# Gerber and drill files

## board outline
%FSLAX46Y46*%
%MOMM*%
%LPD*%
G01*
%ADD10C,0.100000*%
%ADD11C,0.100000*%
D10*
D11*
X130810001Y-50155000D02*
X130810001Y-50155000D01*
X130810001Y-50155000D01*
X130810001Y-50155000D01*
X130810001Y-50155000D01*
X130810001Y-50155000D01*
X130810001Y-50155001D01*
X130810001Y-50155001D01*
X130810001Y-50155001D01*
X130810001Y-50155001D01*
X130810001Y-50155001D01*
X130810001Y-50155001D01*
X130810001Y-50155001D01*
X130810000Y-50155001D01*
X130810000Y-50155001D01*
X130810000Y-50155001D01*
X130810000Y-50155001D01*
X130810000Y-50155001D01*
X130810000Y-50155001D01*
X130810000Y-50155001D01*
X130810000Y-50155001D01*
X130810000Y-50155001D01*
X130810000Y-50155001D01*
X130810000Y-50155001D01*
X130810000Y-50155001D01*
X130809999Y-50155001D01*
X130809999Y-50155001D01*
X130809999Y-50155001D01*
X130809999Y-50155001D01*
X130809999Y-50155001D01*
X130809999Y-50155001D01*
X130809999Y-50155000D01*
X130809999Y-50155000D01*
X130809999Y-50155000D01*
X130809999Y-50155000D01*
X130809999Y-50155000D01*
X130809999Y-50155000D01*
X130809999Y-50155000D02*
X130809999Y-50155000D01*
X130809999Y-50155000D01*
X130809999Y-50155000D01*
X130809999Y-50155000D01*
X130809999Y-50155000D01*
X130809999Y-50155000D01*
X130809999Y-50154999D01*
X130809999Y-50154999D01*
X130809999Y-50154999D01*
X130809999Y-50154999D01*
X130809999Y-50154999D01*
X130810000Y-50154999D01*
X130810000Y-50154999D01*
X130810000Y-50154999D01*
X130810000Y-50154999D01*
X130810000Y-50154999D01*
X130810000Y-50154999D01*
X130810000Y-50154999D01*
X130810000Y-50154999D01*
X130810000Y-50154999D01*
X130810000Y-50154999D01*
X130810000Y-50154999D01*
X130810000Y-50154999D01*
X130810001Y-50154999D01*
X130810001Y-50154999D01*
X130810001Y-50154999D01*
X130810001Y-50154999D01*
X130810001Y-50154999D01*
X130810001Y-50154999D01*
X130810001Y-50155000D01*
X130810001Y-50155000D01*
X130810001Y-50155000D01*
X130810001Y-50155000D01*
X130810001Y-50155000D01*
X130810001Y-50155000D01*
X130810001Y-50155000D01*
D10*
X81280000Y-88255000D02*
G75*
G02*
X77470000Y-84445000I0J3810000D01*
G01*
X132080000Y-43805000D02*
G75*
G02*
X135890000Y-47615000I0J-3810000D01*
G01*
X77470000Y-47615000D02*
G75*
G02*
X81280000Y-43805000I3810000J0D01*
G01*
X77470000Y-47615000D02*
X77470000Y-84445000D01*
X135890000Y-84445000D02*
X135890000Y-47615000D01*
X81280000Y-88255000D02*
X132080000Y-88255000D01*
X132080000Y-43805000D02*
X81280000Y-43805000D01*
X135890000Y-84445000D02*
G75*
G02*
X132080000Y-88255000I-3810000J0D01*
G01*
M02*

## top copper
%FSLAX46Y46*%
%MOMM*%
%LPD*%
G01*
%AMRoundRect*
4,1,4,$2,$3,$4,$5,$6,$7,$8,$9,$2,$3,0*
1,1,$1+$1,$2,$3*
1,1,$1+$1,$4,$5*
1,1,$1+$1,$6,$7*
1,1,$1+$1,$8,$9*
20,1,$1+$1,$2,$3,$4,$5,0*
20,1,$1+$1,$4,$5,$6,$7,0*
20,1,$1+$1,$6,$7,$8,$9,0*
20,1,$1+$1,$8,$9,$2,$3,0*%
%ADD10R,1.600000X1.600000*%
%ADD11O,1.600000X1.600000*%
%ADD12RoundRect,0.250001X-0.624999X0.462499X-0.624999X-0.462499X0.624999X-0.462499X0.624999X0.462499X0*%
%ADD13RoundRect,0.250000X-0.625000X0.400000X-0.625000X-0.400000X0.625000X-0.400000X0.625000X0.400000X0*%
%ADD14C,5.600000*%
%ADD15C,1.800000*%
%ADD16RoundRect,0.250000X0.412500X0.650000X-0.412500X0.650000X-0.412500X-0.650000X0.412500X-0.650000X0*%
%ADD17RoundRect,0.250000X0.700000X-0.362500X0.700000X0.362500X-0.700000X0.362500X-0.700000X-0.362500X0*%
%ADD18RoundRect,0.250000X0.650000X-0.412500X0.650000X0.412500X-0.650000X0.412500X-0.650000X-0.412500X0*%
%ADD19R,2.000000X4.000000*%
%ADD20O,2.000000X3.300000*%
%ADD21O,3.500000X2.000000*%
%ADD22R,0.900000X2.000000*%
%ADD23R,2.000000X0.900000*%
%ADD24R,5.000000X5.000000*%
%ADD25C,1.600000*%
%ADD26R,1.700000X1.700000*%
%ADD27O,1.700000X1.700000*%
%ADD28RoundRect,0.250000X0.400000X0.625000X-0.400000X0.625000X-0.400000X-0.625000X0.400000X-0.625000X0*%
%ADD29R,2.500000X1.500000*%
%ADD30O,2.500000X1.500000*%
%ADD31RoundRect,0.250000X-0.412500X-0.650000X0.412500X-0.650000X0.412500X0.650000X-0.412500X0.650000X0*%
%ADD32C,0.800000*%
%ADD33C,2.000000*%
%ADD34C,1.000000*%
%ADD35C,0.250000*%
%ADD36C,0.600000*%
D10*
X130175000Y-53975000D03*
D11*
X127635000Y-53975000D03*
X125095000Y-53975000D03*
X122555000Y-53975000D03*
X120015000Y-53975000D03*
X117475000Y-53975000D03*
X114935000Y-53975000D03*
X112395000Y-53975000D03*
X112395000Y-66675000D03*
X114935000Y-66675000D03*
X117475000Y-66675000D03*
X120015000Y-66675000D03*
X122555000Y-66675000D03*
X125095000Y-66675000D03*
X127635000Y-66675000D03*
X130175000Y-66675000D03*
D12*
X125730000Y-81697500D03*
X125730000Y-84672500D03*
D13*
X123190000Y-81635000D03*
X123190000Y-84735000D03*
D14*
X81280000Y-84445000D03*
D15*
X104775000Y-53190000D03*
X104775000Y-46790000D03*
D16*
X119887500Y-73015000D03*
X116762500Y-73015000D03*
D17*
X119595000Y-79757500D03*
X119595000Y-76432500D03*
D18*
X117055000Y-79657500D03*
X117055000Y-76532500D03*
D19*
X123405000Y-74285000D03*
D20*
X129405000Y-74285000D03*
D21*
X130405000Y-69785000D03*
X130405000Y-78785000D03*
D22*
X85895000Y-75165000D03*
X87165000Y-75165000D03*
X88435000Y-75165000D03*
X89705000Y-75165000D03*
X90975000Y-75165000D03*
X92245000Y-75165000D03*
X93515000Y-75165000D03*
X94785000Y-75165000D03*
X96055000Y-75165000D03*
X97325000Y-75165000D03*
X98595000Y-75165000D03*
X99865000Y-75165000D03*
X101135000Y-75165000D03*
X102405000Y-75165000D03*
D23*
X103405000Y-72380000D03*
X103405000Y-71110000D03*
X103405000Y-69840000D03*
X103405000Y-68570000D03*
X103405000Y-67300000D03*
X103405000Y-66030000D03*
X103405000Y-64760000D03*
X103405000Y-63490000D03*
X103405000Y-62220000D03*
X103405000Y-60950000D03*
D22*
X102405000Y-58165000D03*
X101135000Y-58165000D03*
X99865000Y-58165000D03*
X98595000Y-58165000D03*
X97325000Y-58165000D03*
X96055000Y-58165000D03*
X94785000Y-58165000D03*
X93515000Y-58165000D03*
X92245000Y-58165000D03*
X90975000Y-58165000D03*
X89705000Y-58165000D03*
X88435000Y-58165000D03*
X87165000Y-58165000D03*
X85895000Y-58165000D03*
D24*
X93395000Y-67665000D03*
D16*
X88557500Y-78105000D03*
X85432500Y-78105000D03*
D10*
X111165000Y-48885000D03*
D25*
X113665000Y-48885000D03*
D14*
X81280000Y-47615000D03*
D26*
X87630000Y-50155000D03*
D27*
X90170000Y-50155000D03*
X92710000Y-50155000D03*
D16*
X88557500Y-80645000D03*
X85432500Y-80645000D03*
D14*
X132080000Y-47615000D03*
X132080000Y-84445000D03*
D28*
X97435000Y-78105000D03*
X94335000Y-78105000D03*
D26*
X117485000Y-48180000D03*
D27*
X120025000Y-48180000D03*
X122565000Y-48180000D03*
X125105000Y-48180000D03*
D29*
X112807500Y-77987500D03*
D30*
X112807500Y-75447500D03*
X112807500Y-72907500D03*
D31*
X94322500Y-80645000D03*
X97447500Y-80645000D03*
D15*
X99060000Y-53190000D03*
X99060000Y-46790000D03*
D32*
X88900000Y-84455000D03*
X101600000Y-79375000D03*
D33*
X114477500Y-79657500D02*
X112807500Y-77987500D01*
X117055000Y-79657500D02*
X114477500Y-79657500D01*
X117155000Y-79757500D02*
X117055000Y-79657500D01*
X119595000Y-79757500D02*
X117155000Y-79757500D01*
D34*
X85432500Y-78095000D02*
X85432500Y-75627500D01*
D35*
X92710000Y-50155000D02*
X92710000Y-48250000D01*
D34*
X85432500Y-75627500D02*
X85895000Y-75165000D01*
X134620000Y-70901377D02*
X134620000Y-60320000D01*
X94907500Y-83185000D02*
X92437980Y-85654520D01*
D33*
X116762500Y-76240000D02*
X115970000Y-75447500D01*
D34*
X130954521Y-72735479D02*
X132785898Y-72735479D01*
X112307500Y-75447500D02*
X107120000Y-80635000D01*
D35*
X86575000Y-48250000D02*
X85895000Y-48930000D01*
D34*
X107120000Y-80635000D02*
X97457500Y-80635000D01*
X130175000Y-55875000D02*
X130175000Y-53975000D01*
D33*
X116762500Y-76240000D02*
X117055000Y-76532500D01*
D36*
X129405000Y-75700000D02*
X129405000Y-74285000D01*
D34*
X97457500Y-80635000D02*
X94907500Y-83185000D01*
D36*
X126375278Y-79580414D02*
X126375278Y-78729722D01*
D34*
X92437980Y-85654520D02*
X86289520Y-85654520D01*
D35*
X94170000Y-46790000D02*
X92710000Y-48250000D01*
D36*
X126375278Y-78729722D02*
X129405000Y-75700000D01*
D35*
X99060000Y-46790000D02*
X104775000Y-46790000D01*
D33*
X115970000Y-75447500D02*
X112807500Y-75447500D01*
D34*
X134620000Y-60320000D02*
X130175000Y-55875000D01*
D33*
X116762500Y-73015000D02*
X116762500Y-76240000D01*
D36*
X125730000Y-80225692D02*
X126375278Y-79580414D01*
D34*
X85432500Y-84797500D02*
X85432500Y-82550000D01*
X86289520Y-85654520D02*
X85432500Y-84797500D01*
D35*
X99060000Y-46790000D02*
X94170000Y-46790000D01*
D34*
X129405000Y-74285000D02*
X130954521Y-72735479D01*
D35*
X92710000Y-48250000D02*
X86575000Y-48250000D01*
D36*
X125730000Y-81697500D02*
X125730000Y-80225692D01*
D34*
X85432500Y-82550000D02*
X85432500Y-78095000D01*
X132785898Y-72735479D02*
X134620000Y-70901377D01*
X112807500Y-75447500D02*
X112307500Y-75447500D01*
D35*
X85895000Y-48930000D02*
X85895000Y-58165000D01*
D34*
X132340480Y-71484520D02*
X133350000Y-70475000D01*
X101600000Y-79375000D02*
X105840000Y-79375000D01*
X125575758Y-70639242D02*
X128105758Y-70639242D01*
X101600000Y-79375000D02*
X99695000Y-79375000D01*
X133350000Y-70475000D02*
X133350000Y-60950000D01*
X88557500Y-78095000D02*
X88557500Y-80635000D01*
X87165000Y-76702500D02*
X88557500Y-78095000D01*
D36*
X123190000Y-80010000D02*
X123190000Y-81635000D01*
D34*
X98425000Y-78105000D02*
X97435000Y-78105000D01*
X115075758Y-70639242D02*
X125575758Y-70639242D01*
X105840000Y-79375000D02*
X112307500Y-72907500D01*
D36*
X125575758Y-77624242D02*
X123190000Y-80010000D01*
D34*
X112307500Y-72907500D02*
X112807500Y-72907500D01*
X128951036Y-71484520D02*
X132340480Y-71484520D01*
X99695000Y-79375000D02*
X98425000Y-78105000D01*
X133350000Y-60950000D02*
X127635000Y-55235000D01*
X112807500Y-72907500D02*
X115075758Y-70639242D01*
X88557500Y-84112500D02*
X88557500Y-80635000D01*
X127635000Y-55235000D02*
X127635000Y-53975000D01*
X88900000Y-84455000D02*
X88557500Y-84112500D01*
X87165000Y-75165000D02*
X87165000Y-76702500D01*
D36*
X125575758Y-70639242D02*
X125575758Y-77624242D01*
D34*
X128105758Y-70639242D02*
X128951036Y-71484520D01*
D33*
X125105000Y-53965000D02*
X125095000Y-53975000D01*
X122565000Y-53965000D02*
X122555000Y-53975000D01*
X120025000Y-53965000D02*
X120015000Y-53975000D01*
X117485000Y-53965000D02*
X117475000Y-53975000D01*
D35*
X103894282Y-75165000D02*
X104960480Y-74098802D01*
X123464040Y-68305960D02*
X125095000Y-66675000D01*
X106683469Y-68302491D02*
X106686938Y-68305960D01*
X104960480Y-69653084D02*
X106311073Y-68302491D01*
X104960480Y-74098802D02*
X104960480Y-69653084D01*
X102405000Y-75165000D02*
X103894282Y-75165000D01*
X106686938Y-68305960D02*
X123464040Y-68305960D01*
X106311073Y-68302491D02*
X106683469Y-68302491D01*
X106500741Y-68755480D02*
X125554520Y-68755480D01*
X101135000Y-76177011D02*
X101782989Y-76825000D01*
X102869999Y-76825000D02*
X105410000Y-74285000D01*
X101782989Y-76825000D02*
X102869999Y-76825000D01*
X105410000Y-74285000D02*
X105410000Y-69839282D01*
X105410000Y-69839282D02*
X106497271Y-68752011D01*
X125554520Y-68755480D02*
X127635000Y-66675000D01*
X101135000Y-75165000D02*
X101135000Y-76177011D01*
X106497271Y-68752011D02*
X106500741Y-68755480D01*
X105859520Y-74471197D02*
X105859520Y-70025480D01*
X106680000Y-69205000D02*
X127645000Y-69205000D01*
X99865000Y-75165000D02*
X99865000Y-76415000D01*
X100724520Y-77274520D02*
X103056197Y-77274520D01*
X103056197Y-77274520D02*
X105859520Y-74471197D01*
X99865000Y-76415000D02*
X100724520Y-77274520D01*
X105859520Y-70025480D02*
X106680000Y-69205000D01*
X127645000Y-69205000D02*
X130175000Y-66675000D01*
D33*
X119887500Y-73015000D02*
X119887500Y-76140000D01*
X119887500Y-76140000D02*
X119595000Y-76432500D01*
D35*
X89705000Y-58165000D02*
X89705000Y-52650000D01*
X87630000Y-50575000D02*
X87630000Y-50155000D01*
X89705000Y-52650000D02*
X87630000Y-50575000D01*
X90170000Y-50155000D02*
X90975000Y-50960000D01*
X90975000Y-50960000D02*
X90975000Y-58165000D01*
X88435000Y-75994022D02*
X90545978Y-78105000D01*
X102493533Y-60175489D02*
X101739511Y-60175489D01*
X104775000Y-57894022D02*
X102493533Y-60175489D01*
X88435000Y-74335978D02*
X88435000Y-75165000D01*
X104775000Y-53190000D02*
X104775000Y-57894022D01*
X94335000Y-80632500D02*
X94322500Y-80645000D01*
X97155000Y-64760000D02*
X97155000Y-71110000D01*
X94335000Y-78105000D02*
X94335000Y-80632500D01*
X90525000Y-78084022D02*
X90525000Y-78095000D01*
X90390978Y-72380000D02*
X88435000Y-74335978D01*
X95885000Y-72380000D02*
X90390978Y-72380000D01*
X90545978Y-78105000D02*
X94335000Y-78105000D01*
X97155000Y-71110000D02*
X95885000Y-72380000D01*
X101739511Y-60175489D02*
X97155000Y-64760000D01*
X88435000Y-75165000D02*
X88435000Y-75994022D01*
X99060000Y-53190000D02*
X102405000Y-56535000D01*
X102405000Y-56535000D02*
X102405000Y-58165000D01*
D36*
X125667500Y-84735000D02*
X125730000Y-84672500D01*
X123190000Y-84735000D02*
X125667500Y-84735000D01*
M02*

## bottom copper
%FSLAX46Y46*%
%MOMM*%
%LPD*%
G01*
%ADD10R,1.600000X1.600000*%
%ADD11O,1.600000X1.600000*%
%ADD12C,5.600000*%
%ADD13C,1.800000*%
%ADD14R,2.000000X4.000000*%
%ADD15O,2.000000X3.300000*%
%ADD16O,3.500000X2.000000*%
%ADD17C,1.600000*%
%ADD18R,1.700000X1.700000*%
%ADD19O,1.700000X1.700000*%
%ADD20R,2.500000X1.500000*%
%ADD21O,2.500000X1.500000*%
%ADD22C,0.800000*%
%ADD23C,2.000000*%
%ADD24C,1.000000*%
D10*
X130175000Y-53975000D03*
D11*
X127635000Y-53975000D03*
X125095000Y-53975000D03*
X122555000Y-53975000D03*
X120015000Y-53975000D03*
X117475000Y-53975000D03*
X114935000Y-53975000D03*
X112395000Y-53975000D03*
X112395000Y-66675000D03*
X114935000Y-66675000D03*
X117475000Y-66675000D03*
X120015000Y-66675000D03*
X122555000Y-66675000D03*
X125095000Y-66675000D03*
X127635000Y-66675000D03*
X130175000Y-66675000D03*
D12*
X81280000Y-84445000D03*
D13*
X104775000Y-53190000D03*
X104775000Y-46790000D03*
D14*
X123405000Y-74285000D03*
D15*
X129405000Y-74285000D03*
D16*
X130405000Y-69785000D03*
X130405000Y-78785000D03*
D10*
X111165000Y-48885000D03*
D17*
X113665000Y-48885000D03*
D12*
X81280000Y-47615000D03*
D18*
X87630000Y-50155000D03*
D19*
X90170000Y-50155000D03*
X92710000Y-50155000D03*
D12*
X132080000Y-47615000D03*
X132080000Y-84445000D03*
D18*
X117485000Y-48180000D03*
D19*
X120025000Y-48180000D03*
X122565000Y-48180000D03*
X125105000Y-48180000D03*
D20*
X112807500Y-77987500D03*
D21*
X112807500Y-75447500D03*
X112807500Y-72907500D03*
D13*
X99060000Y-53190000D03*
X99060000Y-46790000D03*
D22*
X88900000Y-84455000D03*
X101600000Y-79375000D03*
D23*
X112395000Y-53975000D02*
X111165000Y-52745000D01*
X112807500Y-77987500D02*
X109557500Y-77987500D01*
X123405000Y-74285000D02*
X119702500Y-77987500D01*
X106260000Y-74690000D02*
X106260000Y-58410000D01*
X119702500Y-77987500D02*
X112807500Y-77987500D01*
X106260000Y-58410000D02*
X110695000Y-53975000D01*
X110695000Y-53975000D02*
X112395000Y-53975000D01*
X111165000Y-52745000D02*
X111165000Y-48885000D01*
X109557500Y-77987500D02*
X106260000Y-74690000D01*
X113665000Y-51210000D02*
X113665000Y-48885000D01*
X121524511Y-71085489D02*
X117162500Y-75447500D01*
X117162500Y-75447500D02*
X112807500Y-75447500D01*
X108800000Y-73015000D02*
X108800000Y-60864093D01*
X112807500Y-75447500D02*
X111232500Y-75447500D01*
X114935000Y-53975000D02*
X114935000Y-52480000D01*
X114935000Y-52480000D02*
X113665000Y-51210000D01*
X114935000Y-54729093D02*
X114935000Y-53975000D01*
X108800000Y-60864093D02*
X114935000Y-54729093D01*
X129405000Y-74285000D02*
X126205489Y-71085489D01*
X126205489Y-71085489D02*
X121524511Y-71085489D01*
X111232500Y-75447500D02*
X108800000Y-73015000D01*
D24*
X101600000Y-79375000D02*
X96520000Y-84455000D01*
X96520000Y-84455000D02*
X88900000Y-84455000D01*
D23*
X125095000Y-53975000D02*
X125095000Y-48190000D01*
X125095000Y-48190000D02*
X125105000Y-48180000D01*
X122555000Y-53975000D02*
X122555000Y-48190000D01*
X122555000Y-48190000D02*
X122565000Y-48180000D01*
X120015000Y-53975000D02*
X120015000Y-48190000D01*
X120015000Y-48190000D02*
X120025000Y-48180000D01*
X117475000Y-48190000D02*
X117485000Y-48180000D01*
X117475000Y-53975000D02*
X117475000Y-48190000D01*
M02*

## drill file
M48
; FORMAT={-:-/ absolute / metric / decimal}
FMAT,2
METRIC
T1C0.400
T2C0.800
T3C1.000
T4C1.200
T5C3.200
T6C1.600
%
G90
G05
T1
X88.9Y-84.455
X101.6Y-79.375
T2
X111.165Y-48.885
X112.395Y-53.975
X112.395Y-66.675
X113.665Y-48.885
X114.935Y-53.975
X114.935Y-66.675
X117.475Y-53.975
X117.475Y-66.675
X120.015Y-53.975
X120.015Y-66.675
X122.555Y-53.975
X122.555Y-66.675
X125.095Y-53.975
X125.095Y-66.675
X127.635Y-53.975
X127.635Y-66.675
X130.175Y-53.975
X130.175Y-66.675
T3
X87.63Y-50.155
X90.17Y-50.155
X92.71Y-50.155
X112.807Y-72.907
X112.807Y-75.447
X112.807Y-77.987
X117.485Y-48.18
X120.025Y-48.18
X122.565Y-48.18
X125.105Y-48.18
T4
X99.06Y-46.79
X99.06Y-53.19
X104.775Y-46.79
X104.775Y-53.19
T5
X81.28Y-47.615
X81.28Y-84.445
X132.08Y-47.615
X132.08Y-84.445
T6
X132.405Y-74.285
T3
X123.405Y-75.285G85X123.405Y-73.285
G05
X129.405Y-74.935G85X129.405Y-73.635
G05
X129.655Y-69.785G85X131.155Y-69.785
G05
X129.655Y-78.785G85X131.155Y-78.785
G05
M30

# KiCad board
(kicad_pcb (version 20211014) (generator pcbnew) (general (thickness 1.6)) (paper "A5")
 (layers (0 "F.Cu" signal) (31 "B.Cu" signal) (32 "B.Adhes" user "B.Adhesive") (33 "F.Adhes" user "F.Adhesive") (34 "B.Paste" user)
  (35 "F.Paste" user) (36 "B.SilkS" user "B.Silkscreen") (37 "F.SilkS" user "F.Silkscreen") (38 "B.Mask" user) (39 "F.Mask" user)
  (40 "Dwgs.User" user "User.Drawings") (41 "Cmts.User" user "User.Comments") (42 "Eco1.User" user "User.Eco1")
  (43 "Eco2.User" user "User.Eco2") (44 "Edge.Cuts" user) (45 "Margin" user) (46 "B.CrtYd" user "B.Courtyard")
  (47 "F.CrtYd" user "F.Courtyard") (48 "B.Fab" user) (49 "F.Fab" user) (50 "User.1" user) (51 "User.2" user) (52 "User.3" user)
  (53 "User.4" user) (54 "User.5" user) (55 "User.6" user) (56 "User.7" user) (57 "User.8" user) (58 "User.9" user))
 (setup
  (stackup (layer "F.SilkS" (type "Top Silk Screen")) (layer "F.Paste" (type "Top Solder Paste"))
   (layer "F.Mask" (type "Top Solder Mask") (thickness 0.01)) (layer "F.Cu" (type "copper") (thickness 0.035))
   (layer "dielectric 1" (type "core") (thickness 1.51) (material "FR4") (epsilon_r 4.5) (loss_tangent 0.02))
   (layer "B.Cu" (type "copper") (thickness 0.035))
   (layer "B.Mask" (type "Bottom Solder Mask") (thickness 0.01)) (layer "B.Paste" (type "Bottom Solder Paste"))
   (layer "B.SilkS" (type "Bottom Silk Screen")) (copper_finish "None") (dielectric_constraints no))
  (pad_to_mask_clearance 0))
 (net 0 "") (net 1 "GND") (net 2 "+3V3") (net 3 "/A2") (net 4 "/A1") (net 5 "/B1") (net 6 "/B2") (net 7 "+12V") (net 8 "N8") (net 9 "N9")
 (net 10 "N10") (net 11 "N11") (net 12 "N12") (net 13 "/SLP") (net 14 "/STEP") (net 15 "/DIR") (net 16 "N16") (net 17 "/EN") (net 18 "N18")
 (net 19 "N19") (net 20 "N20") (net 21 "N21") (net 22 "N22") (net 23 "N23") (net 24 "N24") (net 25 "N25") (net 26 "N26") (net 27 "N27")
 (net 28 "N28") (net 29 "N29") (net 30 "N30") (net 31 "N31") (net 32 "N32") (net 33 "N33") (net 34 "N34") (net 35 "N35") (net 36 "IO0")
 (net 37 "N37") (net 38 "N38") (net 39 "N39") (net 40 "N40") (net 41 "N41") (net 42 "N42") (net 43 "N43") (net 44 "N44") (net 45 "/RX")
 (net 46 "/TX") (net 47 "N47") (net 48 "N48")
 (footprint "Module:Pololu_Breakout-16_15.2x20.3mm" (layer "F.Cu") (at 130.175 53.975 -90)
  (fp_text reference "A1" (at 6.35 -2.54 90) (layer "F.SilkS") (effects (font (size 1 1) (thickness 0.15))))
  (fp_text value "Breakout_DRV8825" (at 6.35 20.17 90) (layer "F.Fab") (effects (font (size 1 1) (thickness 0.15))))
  (pad "1" thru_hole rect (at 0 0 270) (size 1.6 1.6) (drill 0.8) (layers *.Cu *.Mask) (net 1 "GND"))
  (pad "2" thru_hole oval (at 0 2.54 270) (size 1.6 1.6) (drill 0.8) (layers *.Cu *.Mask) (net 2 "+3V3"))
  (pad "3" thru_hole oval (at 0 5.08 270) (size 1.6 1.6) (drill 0.8) (layers *.Cu *.Mask) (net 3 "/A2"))
  (pad "4" thru_hole oval (at 0 7.62 270) (size 1.6 1.6) (drill 0.8) (layers *.Cu *.Mask) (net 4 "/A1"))
  (pad "5" thru_hole oval (at 0 10.16 270) (size 1.6 1.6) (drill 0.8) (layers *.Cu *.Mask) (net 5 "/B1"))
  (pad "6" thru_hole oval (at 0 12.7 270) (size 1.6 1.6) (drill 0.8) (layers *.Cu *.Mask) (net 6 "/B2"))
  (pad "7" thru_hole oval (at 0 15.24 270) (size 1.6 1.6) (drill 0.8) (layers *.Cu *.Mask) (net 1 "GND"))
  (pad "8" thru_hole oval (at 0 17.78 270) (size 1.6 1.6) (drill 0.8) (layers *.Cu *.Mask) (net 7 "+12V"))
  (pad "9" thru_hole oval (at 12.7 17.78 270) (size 1.6 1.6) (drill 0.8) (layers *.Cu *.Mask) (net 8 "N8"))
  (pad "10" thru_hole oval (at 12.7 15.24 270) (size 1.6 1.6) (drill 0.8) (layers *.Cu *.Mask) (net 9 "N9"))
  (pad "11" thru_hole oval (at 12.7 12.7 270) (size 1.6 1.6) (drill 0.8) (layers *.Cu *.Mask) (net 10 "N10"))
  (pad "12" thru_hole oval (at 12.7 10.16 270) (size 1.6 1.6) (drill 0.8) (layers *.Cu *.Mask) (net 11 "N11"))
  (pad "13" thru_hole oval (at 12.7 7.62 270) (size 1.6 1.6) (drill 0.8) (layers *.Cu *.Mask) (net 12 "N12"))
  (pad "14" thru_hole oval (at 12.7 5.08 270) (size 1.6 1.6) (drill 0.8) (layers *.Cu *.Mask) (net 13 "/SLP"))
  (pad "15" thru_hole oval (at 12.7 2.54 270) (size 1.6 1.6) (drill 0.8) (layers *.Cu *.Mask) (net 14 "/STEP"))
  (pad "16" thru_hole oval (at 12.7 0 270) (size 1.6 1.6) (drill 0.8) (layers *.Cu *.Mask) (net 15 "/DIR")))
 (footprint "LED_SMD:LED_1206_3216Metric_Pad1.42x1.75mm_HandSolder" (layer "F.Cu") (at 125.73 83.185 -90)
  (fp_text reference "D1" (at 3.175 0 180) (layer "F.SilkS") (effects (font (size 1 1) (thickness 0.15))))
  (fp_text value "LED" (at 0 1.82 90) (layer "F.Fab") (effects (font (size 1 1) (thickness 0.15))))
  (pad "1" smd roundrect (at -1.4875 0 270) (size 1.425 1.75) (layers "F.Cu" "F.Paste" "F.Mask") (roundrect_rratio 0.175439) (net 1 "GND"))
  (pad "2" smd roundrect (at 1.4875 0 270) (size 1.425 1.75) (layers "F.Cu" "F.Paste" "F.Mask") (roundrect_rratio 0.175439) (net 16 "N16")))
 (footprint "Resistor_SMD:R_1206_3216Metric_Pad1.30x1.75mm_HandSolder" (layer "F.Cu") (at 123.19 83.185 -90)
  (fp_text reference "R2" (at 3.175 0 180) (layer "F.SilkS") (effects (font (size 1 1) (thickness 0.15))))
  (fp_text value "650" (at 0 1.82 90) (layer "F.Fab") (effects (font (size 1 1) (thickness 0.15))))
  (pad "1" smd roundrect (at -1.55 0 270) (size 1.3 1.75) (layers "F.Cu" "F.Paste" "F.Mask") (roundrect_rratio 0.192308) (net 2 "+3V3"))
  (pad "2" smd roundrect (at 1.55 0 270) (size 1.3 1.75) (layers "F.Cu" "F.Paste" "F.Mask") (roundrect_rratio 0.192308) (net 16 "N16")))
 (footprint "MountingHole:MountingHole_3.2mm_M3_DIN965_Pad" (layer "F.Cu") (at 81.28 84.445)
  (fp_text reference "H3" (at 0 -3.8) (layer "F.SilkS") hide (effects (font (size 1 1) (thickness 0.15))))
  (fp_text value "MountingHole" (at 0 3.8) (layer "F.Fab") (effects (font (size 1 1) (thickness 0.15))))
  (pad "1" thru_hole circle (at 0 0) (size 5.6 5.6) (drill 3.2) (layers *.Cu *.Mask)))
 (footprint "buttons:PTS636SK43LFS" (layer "F.Cu") (at 104.775 53.19 90)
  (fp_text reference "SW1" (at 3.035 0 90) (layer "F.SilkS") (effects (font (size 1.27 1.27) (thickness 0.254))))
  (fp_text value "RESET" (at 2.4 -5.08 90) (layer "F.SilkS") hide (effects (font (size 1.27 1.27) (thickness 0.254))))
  (pad "1" thru_hole circle (at 0 0 90) (size 1.8 1.8) (drill 1.2) (layers *.Cu *.Mask) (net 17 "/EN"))
  (pad "2" thru_hole circle (at 6.4 0 90) (size 1.8 1.8) (drill 1.2) (layers *.Cu *.Mask) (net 1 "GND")))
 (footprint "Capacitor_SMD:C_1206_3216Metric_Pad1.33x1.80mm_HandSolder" (layer "F.Cu") (at 118.325 73.015 180)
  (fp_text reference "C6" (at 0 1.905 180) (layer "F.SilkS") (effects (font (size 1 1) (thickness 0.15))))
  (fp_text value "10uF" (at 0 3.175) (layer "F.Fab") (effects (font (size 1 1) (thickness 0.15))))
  (pad "1" smd roundrect (at -1.5625 0 180) (size 1.325 1.8) (layers "F.Cu" "F.Paste" "F.Mask") (roundrect_rratio 0.188679) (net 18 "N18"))
  (pad "2" smd roundrect (at 1.5625 0 180) (size 1.325 1.8) (layers "F.Cu" "F.Paste" "F.Mask") (roundrect_rratio 0.188679) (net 1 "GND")))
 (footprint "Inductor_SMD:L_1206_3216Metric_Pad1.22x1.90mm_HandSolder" (layer "F.Cu") (at 119.595 78.095 90)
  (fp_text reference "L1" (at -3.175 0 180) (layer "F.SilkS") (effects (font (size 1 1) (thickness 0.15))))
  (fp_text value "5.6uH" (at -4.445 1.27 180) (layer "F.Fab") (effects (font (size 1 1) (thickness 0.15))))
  (pad "1" smd roundrect (at -1.6625 0 90) (size 1.225 1.9) (layers "F.Cu" "F.Paste" "F.Mask") (roundrect_rratio 0.204082) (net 7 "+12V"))
  (pad "2" smd roundrect (at 1.6625 0 90) (size 1.225 1.9) (layers "F.Cu" "F.Paste" "F.Mask") (roundrect_rratio 0.204082) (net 18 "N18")))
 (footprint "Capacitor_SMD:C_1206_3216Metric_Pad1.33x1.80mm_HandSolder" (layer "F.Cu") (at 117.055 78.095 90)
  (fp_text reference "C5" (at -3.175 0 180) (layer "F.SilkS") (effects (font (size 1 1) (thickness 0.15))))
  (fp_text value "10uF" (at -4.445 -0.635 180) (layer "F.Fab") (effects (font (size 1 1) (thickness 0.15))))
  (pad "1" smd roundrect (at -1.5625 0 90) (size 1.325 1.8) (layers "F.Cu" "F.Paste" "F.Mask") (roundrect_rratio 0.188679) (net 7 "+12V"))
  (pad "2" smd roundrect (at 1.5625 0 90) (size 1.325 1.8) (layers "F.Cu" "F.Paste" "F.Mask") (roundrect_rratio 0.188679) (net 1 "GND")))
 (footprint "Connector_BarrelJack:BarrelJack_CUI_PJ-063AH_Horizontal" (layer "F.Cu") (at 123.405 74.285 90)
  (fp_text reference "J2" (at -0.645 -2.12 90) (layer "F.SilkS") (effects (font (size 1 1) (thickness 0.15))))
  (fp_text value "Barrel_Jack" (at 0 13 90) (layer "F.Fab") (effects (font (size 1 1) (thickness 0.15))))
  (pad "" np_thru_hole circle (at 0 9 90) (size 1.6 1.6) (drill 1.6) (layers *.Cu *.Mask))
  (pad "1" thru_hole rect (at 0 0 90) (size 4 2) (drill oval 3 1) (layers *.Cu *.Mask) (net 7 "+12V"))
  (pad "2" thru_hole oval (at 0 6 90) (size 3.3 2) (drill oval 2.3 1) (layers *.Cu *.Mask) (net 1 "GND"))
  (pad "MP" thru_hole oval (at 4.5 7 90) (size 2 3.5) (drill oval 1 2.5) (layers *.Cu *.Mask))
  (pad "MP" thru_hole oval (at -4.5 7 90) (size 2 3.5) (drill oval 1 2.5) (layers *.Cu *.Mask)))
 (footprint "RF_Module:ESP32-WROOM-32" (layer "F.Cu") (at 94.15 66.665 90)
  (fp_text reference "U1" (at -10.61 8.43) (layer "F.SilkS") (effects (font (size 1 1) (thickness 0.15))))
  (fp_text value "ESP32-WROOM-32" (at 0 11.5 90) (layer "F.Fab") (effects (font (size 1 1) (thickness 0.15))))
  (pad "1" smd rect (at -8.5 -8.255 90) (size 2 0.9) (layers "F.Cu" "F.Paste" "F.Mask") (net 1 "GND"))
  (pad "2" smd rect (at -8.5 -6.985 90) (size 2 0.9) (layers "F.Cu" "F.Paste" "F.Mask") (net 2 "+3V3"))
  (pad "3" smd rect (at -8.5 -5.715 90) (size 2 0.9) (layers "F.Cu" "F.Paste" "F.Mask") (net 17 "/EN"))
  (pad "4" smd rect (at -8.5 -4.445 90) (size 2 0.9) (layers "F.Cu" "F.Paste" "F.Mask") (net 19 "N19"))
  (pad "5" smd rect (at -8.5 -3.175 90) (size 2 0.9) (layers "F.Cu" "F.Paste" "F.Mask") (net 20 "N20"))
  (pad "6" smd rect (at -8.5 -1.905 90) (size 2 0.9) (layers "F.Cu" "F.Paste" "F.Mask") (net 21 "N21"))
  (pad "7" smd rect (at -8.5 -0.635 90) (size 2 0.9) (layers "F.Cu" "F.Paste" "F.Mask") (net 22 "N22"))
  (pad "8" smd rect (at -8.5 0.635 90) (size 2 0.9) (layers "F.Cu" "F.Paste" "F.Mask") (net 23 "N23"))
  (pad "9" smd rect (at -8.5 1.905 90) (size 2 0.9) (layers "F.Cu" "F.Paste" "F.Mask") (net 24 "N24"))
  (pad "10" smd rect (at -8.5 3.175 90) (size 2 0.9) (layers "F.Cu" "F.Paste" "F.Mask") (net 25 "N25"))
  (pad "11" smd rect (at -8.5 4.445 90) (size 2 0.9) (layers "F.Cu" "F.Paste" "F.Mask") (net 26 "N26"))
  (pad "12" smd rect (at -8.5 5.715 90) (size 2 0.9) (layers "F.Cu" "F.Paste" "F.Mask") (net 15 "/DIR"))
  (pad "13" smd rect (at -8.5 6.985 90) (size 2 0.9) (layers "F.Cu" "F.Paste" "F.Mask") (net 14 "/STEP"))
  (pad "14" smd rect (at -8.5 8.255 90) (size 2 0.9) (layers "F.Cu" "F.Paste" "F.Mask") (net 13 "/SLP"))
  (pad "15" smd rect (at -5.715 9.255 180) (size 2 0.9) (layers "F.Cu" "F.Paste" "F.Mask") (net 1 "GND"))
  (pad "16" smd rect (at -4.445 9.255 180) (size 2 0.9) (layers "F.Cu" "F.Paste" "F.Mask") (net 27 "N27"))
  (pad "17" smd rect (at -3.175 9.255 180) (size 2 0.9) (layers "F.Cu" "F.Paste" "F.Mask") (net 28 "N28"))
  (pad "18" smd rect (at -1.905 9.255 180) (size 2 0.9) (layers "F.Cu" "F.Paste" "F.Mask") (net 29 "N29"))
  (pad "19" smd rect (at -0.635 9.255 180) (size 2 0.9) (layers "F.Cu" "F.Paste" "F.Mask") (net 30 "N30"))
  (pad "20" smd rect (at 0.635 9.255 180) (size 2 0.9) (layers "F.Cu" "F.Paste" "F.Mask") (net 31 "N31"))
  (pad "21" smd rect (at 1.905 9.255 180) (size 2 0.9) (layers "F.Cu" "F.Paste" "F.Mask") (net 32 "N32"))
  (pad "22" smd rect (at 3.175 9.255 180) (size 2 0.9) (layers "F.Cu" "F.Paste" "F.Mask") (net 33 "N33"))
  (pad "23" smd rect (at 4.445 9.255 180) (size 2 0.9) (layers "F.Cu" "F.Paste" "F.Mask") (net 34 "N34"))
  (pad "24" smd rect (at 5.715 9.255 180) (size 2 0.9) (layers "F.Cu" "F.Paste" "F.Mask") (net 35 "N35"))
  (pad "25" smd rect (at 8.5 8.255 90) (size 2 0.9) (layers "F.Cu" "F.Paste" "F.Mask") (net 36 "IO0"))
  (pad "26" smd rect (at 8.5 6.985 90) (size 2 0.9) (layers "F.Cu" "F.Paste" "F.Mask") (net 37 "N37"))
  (pad "27" smd rect (at 8.5 5.715 90) (size 2 0.9) (layers "F.Cu" "F.Paste" "F.Mask") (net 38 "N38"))
  (pad "28" smd rect (at 8.5 4.445 90) (size 2 0.9) (layers "F.Cu" "F.Paste" "F.Mask") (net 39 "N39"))
  (pad "29" smd rect (at 8.5 3.175 90) (size 2 0.9) (layers "F.Cu" "F.Paste" "F.Mask") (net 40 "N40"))
  (pad "30" smd rect (at 8.5 1.905 90) (size 2 0.9) (layers "F.Cu" "F.Paste" "F.Mask") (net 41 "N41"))
  (pad "31" smd rect (at 8.5 0.635 90) (size 2 0.9) (layers "F.Cu" "F.Paste" "F.Mask") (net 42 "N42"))
  (pad "32" smd rect (at 8.5 -0.635 90) (size 2 0.9) (layers "F.Cu" "F.Paste" "F.Mask") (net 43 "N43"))
  (pad "33" smd rect (at 8.5 -1.905 90) (size 2 0.9) (layers "F.Cu" "F.Paste" "F.Mask") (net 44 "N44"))
  (pad "34" smd rect (at 8.5 -3.175 90) (size 2 0.9) (layers "F.Cu" "F.Paste" "F.Mask") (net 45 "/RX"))
  (pad "35" smd rect (at 8.5 -4.445 90) (size 2 0.9) (layers "F.Cu" "F.Paste" "F.Mask") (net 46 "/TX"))
  (pad "36" smd rect (at 8.5 -5.715 90) (size 2 0.9) (layers "F.Cu" "F.Paste" "F.Mask") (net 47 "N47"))
  (pad "37" smd rect (at 8.5 -6.985 90) (size 2 0.9) (layers "F.Cu" "F.Paste" "F.Mask") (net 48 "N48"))
  (pad "38" smd rect (at 8.5 -8.255 90) (size 2 0.9) (layers "F.Cu" "F.Paste" "F.Mask") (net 1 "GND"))
  (pad "39" smd rect (at -1 -0.755 90) (size 5 5) (layers "F.Cu" "F.Paste" "F.Mask") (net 1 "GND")))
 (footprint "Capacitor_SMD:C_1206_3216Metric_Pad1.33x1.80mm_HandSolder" (layer "F.Cu") (at 86.995 78.105 180)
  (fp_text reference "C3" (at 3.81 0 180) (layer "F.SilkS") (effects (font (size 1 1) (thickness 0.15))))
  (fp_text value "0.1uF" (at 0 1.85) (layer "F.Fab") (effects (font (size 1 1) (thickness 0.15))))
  (pad "1" smd roundrect (at -1.5625 0 180) (size 1.325 1.8) (layers "F.Cu" "F.Paste" "F.Mask") (roundrect_rratio 0.188679) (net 2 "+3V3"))
  (pad "2" smd roundrect (at 1.5625 0 180) (size 1.325 1.8) (layers "F.Cu" "F.Paste" "F.Mask") (roundrect_rratio 0.188679) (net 1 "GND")))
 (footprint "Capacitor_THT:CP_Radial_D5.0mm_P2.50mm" (layer "F.Cu") (at 111.165 48.885)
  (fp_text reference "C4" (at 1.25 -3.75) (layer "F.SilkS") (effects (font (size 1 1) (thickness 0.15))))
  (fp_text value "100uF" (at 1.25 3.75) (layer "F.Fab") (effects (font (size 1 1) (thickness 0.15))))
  (pad "1" thru_hole rect (at 0 0) (size 1.6 1.6) (drill 0.8) (layers *.Cu *.Mask) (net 7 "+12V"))
  (pad "2" thru_hole circle (at 2.5 0) (size 1.6 1.6) (drill 0.8) (layers *.Cu *.Mask) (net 1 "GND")))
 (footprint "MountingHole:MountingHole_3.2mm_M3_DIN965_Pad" (layer "F.Cu") (at 81.28 47.615)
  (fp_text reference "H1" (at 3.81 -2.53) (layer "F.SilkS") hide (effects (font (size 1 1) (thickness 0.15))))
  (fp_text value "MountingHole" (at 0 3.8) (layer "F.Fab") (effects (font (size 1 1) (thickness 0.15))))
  (pad "1" thru_hole circle (at 0 0) (size 5.6 5.6) (drill 3.2) (layers *.Cu *.Mask)))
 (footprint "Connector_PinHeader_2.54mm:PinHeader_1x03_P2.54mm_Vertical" (layer "F.Cu") (at 87.63 50.155 90)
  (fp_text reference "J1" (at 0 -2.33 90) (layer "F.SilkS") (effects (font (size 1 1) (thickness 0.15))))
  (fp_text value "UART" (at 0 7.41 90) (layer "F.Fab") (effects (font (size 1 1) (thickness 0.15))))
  (pad "1" thru_hole rect (at 0 0 90) (size 1.7 1.7) (drill 1) (layers *.Cu *.Mask) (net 46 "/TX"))
  (pad "2" thru_hole oval (at 0 2.54 90) (size 1.7 1.7) (drill 1) (layers *.Cu *.Mask) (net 45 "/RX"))
  (pad "3" thru_hole oval (at 0 5.08 90) (size 1.7 1.7) (drill 1) (layers *.Cu *.Mask) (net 1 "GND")))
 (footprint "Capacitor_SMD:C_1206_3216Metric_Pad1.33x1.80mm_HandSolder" (layer "F.Cu") (at 86.995 80.645 180)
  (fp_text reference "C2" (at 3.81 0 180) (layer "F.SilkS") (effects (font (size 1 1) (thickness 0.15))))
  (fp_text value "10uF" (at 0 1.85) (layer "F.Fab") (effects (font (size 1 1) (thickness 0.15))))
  (pad "1" smd roundrect (at -1.5625 0 180) (size 1.325 1.8) (layers "F.Cu" "F.Paste" "F.Mask") (roundrect_rratio 0.188679) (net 2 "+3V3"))
  (pad "2" smd roundrect (at 1.5625 0 180) (size 1.325 1.8) (layers "F.Cu" "F.Paste" "F.Mask") (roundrect_rratio 0.188679) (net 1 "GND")))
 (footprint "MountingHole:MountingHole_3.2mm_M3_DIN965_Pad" (layer "F.Cu") (at 132.08 47.615)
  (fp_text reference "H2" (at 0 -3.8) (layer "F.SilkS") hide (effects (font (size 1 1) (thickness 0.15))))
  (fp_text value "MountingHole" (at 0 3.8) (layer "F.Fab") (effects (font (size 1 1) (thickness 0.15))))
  (pad "1" thru_hole circle (at 0 0) (size 5.6 5.6) (drill 3.2) (layers *.Cu *.Mask)))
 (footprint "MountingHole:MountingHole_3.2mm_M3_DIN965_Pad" (layer "F.Cu") (at 132.08 84.445)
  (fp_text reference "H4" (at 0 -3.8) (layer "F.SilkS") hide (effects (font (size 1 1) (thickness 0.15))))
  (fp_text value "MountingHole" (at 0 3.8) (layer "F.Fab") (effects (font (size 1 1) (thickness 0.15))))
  (pad "1" thru_hole circle (at 0 0) (size 5.6 5.6) (drill 3.2) (layers *.Cu *.Mask)))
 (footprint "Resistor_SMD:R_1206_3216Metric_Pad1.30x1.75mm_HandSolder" (layer "F.Cu") (at 95.885 78.105 180)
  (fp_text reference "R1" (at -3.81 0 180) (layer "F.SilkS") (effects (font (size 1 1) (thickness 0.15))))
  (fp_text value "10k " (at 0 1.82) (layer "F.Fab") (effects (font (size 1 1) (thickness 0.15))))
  (pad "1" smd roundrect (at -1.55 0 180) (size 1.3 1.75) (layers "F.Cu" "F.Paste" "F.Mask") (roundrect_rratio 0.192308) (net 2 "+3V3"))
  (pad "2" smd roundrect (at 1.55 0 180) (size 1.3 1.75) (layers "F.Cu" "F.Paste" "F.Mask") (roundrect_rratio 0.192308) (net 17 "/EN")))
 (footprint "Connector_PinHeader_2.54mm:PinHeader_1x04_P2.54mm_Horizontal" (layer "F.Cu") (at 117.485 48.18 90)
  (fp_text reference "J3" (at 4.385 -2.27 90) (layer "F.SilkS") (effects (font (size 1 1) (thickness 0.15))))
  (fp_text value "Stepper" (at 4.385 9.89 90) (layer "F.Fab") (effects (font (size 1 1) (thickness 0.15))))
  (pad "1" thru_hole rect (at 0 0 90) (size 1.7 1.7) (drill 1) (layers *.Cu *.Mask) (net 6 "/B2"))
  (pad "2" thru_hole oval (at 0 2.54 90) (size 1.7 1.7) (drill 1) (layers *.Cu *.Mask) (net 5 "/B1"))
  (pad "3" thru_hole oval (at 0 5.08 90) (size 1.7 1.7) (drill 1) (layers *.Cu *.Mask) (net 4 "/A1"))
  (pad "4" thru_hole oval (at 0 7.62 90) (size 1.7 1.7) (drill 1) (layers *.Cu *.Mask) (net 3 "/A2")))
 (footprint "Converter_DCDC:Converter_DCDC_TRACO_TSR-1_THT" (layer "F.Cu") (at 112.8075 77.9875 90)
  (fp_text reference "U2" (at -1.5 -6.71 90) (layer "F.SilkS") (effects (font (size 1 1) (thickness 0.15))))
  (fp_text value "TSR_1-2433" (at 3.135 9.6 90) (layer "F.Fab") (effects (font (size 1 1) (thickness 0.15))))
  (pad "1" thru_hole rect (at 0 0 90) (size 1.5 2.5) (drill 1) (layers *.Cu *.Mask) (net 7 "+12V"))
  (pad "2" thru_hole oval (at 2.54 0 90) (size 1.5 2.5) (drill 1) (layers *.Cu *.Mask) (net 1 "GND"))
  (pad "3" thru_hole oval (at 5.08 0 90) (size 1.5 2.5) (drill 1) (layers *.Cu *.Mask) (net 2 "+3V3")))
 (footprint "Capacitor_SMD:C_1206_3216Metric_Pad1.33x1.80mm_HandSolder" (layer "F.Cu") (at 95.885 80.645)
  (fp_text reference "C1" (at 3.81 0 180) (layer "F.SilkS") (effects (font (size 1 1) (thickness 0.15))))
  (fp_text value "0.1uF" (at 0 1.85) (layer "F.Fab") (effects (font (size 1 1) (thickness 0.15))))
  (pad "1" smd roundrect (at -1.5625 0) (size 1.325 1.8) (layers "F.Cu" "F.Paste" "F.Mask") (roundrect_rratio 0.188679) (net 17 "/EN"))
  (pad "2" smd roundrect (at 1.5625 0) (size 1.325 1.8) (layers "F.Cu" "F.Paste" "F.Mask") (roundrect_rratio 0.188679) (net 1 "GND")))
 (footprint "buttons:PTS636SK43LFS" (layer "F.Cu") (at 99.06 53.19 90)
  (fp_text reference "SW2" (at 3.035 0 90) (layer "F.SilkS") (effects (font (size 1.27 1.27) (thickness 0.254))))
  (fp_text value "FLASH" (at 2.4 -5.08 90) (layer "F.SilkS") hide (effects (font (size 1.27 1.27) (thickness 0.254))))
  (pad "1" thru_hole circle (at 0 0 90) (size 1.8 1.8) (drill 1.2) (layers *.Cu *.Mask) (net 36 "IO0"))
  (pad "2" thru_hole circle (at 6.4 0 90) (size 1.8 1.8) (drill 1.2) (layers *.Cu *.Mask) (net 1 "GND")))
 (gr_circle (center 130.81 50.155) (end 130.81 50.155) (layer "Edge.Cuts") (width 0.1) (fill none))
 (gr_arc (start 81.28 88.255) (mid 78.585923 87.139077) (end 77.47 84.445) (layer "Edge.Cuts") (width 0.1))
 (gr_arc (start 132.08 43.805) (mid 134.774077 44.920923) (end 135.89 47.615) (layer "Edge.Cuts") (width 0.1))
 (gr_arc (start 77.47 47.615) (mid 78.585923 44.920923) (end 81.28 43.805) (layer "Edge.Cuts") (width 0.1))
 (gr_line (start 77.47 47.615) (end 77.47 84.445) (layer "Edge.Cuts") (width 0.1))
 (gr_line (start 135.89 84.445) (end 135.89 47.615) (layer "Edge.Cuts") (width 0.1))
 (gr_line (start 81.28 88.255) (end 132.08 88.255) (layer "Edge.Cuts") (width 0.1))
 (gr_line (start 132.08 43.805) (end 81.28 43.805) (layer "Edge.Cuts") (width 0.1))
 (gr_arc (start 135.89 84.445) (mid 134.774077 87.139077) (end 132.08 88.255) (layer "Edge.Cuts") (width 0.1))
 (segment (start 114.4775 79.6575) (end 112.8075 77.9875) (width 2) (layer "F.Cu") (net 7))
 (segment (start 117.055 79.6575) (end 114.4775 79.6575) (width 2) (layer "F.Cu") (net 7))
 (segment (start 117.155 79.7575) (end 117.055 79.6575) (width 2) (layer "F.Cu") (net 7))
 (segment (start 119.595 79.7575) (end 117.155 79.7575) (width 2) (layer "F.Cu") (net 7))
 (segment (start 112.395 53.975) (end 111.165 52.745) (width 2) (layer "B.Cu") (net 7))
 (segment (start 112.8075 77.9875) (end 109.5575 77.9875) (width 2) (layer "B.Cu") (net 7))
 (segment (start 123.405 74.285) (end 119.7025 77.9875) (width 2) (layer "B.Cu") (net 7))
 (segment (start 106.26 74.69) (end 106.26 58.41) (width 2) (layer "B.Cu") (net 7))
 (segment (start 119.7025 77.9875) (end 112.8075 77.9875) (width 2) (layer "B.Cu") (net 7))
 (segment (start 106.26 58.41) (end 110.695 53.975) (width 2) (layer "B.Cu") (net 7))
 (segment (start 110.695 53.975) (end 112.395 53.975) (width 2) (layer "B.Cu") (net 7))
 (segment (start 111.165 52.745) (end 111.165 48.885) (width 2) (layer "B.Cu") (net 7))
 (segment (start 109.5575 77.9875) (end 106.26 74.69) (width 2) (layer "B.Cu") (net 7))
 (segment (start 85.4325 78.095) (end 85.4325 75.6275) (width 1) (layer "F.Cu") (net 1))
 (segment (start 92.71 50.155) (end 92.71 48.25) (width 0.25) (layer "F.Cu") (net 1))
 (segment (start 85.4325 75.6275) (end 85.895 75.165) (width 1) (layer "F.Cu") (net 1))
 (segment (start 134.62 70.901377) (end 134.62 60.32) (width 1) (layer "F.Cu") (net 1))
 (segment (start 94.9075 83.185) (end 92.43798 85.65452) (width 1) (layer "F.Cu") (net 1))
 (segment (start 116.7625 76.24) (end 115.97 75.4475) (width 2) (layer "F.Cu") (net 1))
 (segment (start 130.954521 72.735479) (end 132.785898 72.735479) (width 1) (layer "F.Cu") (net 1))
 (segment (start 112.3075 75.4475) (end 107.12 80.635) (width 1) (layer "F.Cu") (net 1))
 (segment (start 86.575 48.25) (end 85.895 48.93) (width 0.25) (layer "F.Cu") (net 1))
 (segment (start 107.12 80.635) (end 97.4575 80.635) (width 1) (layer "F.Cu") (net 1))
 (segment (start 130.175 55.875) (end 130.175 53.975) (width 1) (layer "F.Cu") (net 1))
 (segment (start 116.7625 76.24) (end 117.055 76.5325) (width 2) (layer "F.Cu") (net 1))
 (segment (start 129.405 75.7) (end 129.405 74.285) (width 0.6) (layer "F.Cu") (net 1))
 (segment (start 97.4575 80.635) (end 94.9075 83.185) (width 1) (layer "F.Cu") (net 1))
 (segment (start 126.375278 79.580414) (end 126.375278 78.729722) (width 0.6) (layer "F.Cu") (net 1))
 (segment (start 92.43798 85.65452) (end 86.28952 85.65452) (width 1) (layer "F.Cu") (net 1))
 (segment (start 94.17 46.79) (end 92.71 48.25) (width 0.25) (layer "F.Cu") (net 1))
 (segment (start 126.375278 78.729722) (end 129.405 75.7) (width 0.6) (layer "F.Cu") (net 1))
 (segment (start 99.06 46.79) (end 104.775 46.79) (width 0.25) (layer "F.Cu") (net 1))
 (segment (start 115.97 75.4475) (end 112.8075 75.4475) (width 2) (layer "F.Cu") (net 1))
 (segment (start 134.62 60.32) (end 130.175 55.875) (width 1) (layer "F.Cu") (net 1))
 (segment (start 116.7625 73.015) (end 116.7625 76.24) (width 2) (layer "F.Cu") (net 1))
 (segment (start 125.73 80.225692) (end 126.375278 79.580414) (width 0.6) (layer "F.Cu") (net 1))
 (segment (start 85.4325 84.7975) (end 85.4325 82.55) (width 1) (layer "F.Cu") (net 1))
 (segment (start 86.28952 85.65452) (end 85.4325 84.7975) (width 1) (layer "F.Cu") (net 1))
 (segment (start 99.06 46.79) (end 94.17 46.79) (width 0.25) (layer "F.Cu") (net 1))
 (segment (start 129.405 74.285) (end 130.954521 72.735479) (width 1) (layer "F.Cu") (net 1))
 (segment (start 92.71 48.25) (end 86.575 48.25) (width 0.25) (layer "F.Cu") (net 1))
 (segment (start 125.73 81.6975) (end 125.73 80.225692) (width 0.6) (layer "F.Cu") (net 1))
 (segment (start 85.4325 82.55) (end 85.4325 78.095) (width 1) (layer "F.Cu") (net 1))
 (segment (start 132.785898 72.735479) (end 134.62 70.901377) (width 1) (layer "F.Cu") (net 1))
 (segment (start 112.8075 75.4475) (end 112.3075 75.4475) (width 1) (layer "F.Cu") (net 1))
 (segment (start 85.895 48.93) (end 85.895 58.165) (width 0.25) (layer "F.Cu") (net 1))
 (segment (start 113.665 51.21) (end 113.665 48.885) (width 2) (layer "B.Cu") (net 1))
 (segment (start 121.524511 71.085489) (end 117.1625 75.4475) (width 2) (layer "B.Cu") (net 1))
 (segment (start 117.1625 75.4475) (end 112.8075 75.4475) (width 2) (layer "B.Cu") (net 1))
 (segment (start 108.8 73.015) (end 108.8 60.864093) (width 2) (layer "B.Cu") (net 1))
 (segment (start 112.8075 75.4475) (end 111.2325 75.4475) (width 2) (layer "B.Cu") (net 1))
 (segment (start 114.935 53.975) (end 114.935 52.48) (width 2) (layer "B.Cu") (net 1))
 (segment (start 114.935 52.48) (end 113.665 51.21) (width 2) (layer "B.Cu") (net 1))
 (segment (start 114.935 54.729093) (end 114.935 53.975) (width 2) (layer "B.Cu") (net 1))
 (segment (start 108.8 60.864093) (end 114.935 54.729093) (width 2) (layer "B.Cu") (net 1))
 (segment (start 129.405 74.285) (end 126.205489 71.085489) (width 2) (layer "B.Cu") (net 1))
 (segment (start 126.205489 71.085489) (end 121.524511 71.085489) (width 2) (layer "B.Cu") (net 1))
 (segment (start 111.2325 75.4475) (end 108.8 73.015) (width 2) (layer "B.Cu") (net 1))
 (segment (start 132.34048 71.48452) (end 133.35 70.475) (width 1) (layer "F.Cu") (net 2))
 (segment (start 101.6 79.375) (end 105.84 79.375) (width 1) (layer "F.Cu") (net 2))
 (segment (start 125.575758 70.639242) (end 128.105758 70.639242) (width 1) (layer "F.Cu") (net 2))
 (segment (start 101.6 79.375) (end 99.695 79.375) (width 1) (layer "F.Cu") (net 2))
 (segment (start 133.35 70.475) (end 133.35 60.95) (width 1) (layer "F.Cu") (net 2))
 (segment (start 88.5575 78.095) (end 88.5575 80.635) (width 1) (layer "F.Cu") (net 2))
 (segment (start 87.165 76.7025) (end 88.5575 78.095) (width 1) (layer "F.Cu") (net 2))
 (segment (start 123.19 80.01) (end 123.19 81.635) (width 0.6) (layer "F.Cu") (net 2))
 (segment (start 98.425 78.105) (end 97.435 78.105) (width 1) (layer "F.Cu") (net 2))
 (segment (start 115.075758 70.639242) (end 125.575758 70.639242) (width 1) (layer "F.Cu") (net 2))
 (segment (start 105.84 79.375) (end 112.3075 72.9075) (width 1) (layer "F.Cu") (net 2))
 (segment (start 125.575758 77.624242) (end 123.19 80.01) (width 0.6) (layer "F.Cu") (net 2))
 (segment (start 112.3075 72.9075) (end 112.8075 72.9075) (width 1) (layer "F.Cu") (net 2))
 (segment (start 128.951036 71.48452) (end 132.34048 71.48452) (width 1) (layer "F.Cu") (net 2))
 (segment (start 99.695 79.375) (end 98.425 78.105) (width 1) (layer "F.Cu") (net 2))
 (segment (start 133.35 60.95) (end 127.635 55.235) (width 1) (layer "F.Cu") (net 2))
 (segment (start 112.8075 72.9075) (end 115.075758 70.639242) (width 1) (layer "F.Cu") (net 2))
 (segment (start 88.5575 84.1125) (end 88.5575 80.635) (width 1) (layer "F.Cu") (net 2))
 (segment (start 127.635 55.235) (end 127.635 53.975) (width 1) (layer "F.Cu") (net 2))
 (segment (start 88.9 84.455) (end 88.5575 84.1125) (width 1) (layer "F.Cu") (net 2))
 (segment (start 87.165 75.165) (end 87.165 76.7025) (width 1) (layer "F.Cu") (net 2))
 (segment (start 125.575758 70.639242) (end 125.575758 77.624242) (width 0.6) (layer "F.Cu") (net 2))
 (segment (start 128.105758 70.639242) (end 128.951036 71.48452) (width 1) (layer "F.Cu") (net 2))
 (via (at 88.9 84.455) (size 0.8) (drill 0.4) (layers "F.Cu" "B.Cu") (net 2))
 (via (at 101.6 79.375) (size 0.8) (drill 0.4) (layers "F.Cu" "B.Cu") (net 2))
 (segment (start 101.6 79.375) (end 96.52 84.455) (width 1) (layer "B.Cu") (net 2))
 (segment (start 96.52 84.455) (end 88.9 84.455) (width 1) (layer "B.Cu") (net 2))
 (segment (start 125.105 53.965) (end 125.095 53.975) (width 2) (layer "F.Cu") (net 3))
 (segment (start 125.095 53.975) (end 125.095 48.19) (width 2) (layer "B.Cu") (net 3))
 (segment (start 125.095 48.19) (end 125.105 48.18) (width 2) (layer "B.Cu") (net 3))
 (segment (start 122.565 53.965) (end 122.555 53.975) (width 2) (layer "F.Cu") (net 4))
 (segment (start 122.555 53.975) (end 122.555 48.19) (width 2) (layer "B.Cu") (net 4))
 (segment (start 122.555 48.19) (end 122.565 48.18) (width 2) (layer "B.Cu") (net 4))
 (segment (start 120.025 53.965) (end 120.015 53.975) (width 2) (layer "F.Cu") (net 5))
 (segment (start 120.015 53.975) (end 120.015 48.19) (width 2) (layer "B.Cu") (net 5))
 (segment (start 120.015 48.19) (end 120.025 48.18) (width 2) (layer "B.Cu") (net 5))
 (segment (start 117.485 53.965) (end 117.475 53.975) (width 2) (layer "F.Cu") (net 6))
 (segment (start 117.475 48.19) (end 117.485 48.18) (width 2) (layer "B.Cu") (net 6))
 (segment (start 117.475 53.975) (end 117.475 48.19) (width 2) (layer "B.Cu") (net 6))
 (segment (start 103.894282 75.165) (end 104.96048 74.098802) (width 0.25) (layer "F.Cu") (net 13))
 (segment (start 123.46404 68.30596) (end 125.095 66.675) (width 0.25) (layer "F.Cu") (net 13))
 (segment (start 106.683469 68.302491) (end 106.686938 68.30596) (width 0.25) (layer "F.Cu") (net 13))
 (segment (start 104.96048 69.653084) (end 106.311073 68.302491) (width 0.25) (layer "F.Cu") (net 13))
 (segment (start 104.96048 74.098802) (end 104.96048 69.653084) (width 0.25) (layer "F.Cu") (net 13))
 (segment (start 102.405 75.165) (end 103.894282 75.165) (width 0.25) (layer "F.Cu") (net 13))
 (segment (start 106.686938 68.30596) (end 123.46404 68.30596) (width 0.25) (layer "F.Cu") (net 13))
 (segment (start 106.311073 68.302491) (end 106.683469 68.302491) (width 0.25) (layer "F.Cu") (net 13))
 (segment (start 106.500741 68.75548) (end 125.55452 68.75548) (width 0.25) (layer "F.Cu") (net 14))
 (segment (start 101.135 76.177011) (end 101.782989 76.825) (width 0.25) (layer "F.Cu") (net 14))
 (segment (start 102.869999 76.825) (end 105.41 74.285) (width 0.25) (layer "F.Cu") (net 14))
 (segment (start 101.782989 76.825) (end 102.869999 76.825) (width 0.25) (layer "F.Cu") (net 14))
 (segment (start 105.41 74.285) (end 105.41 69.839282) (width 0.25) (layer "F.Cu") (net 14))
 (segment (start 105.41 69.839282) (end 106.497271 68.752011) (width 0.25) (layer "F.Cu") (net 14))
 (segment (start 125.55452 68.75548) (end 127.635 66.675) (width 0.25) (layer "F.Cu") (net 14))
 (segment (start 101.135 75.165) (end 101.135 76.177011) (width 0.25) (layer "F.Cu") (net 14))
 (segment (start 106.497271 68.752011) (end 106.500741 68.75548) (width 0.25) (layer "F.Cu") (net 14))
 (segment (start 105.85952 74.471197) (end 105.85952 70.02548) (width 0.25) (layer "F.Cu") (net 15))
 (segment (start 106.68 69.205) (end 127.645 69.205) (width 0.25) (layer "F.Cu") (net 15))
 (segment (start 99.865 75.165) (end 99.865 76.415) (width 0.25) (layer "F.Cu") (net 15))
 (segment (start 100.72452 77.27452) (end 103.056197 77.27452) (width 0.25) (layer "F.Cu") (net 15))
 (segment (start 103.056197 77.27452) (end 105.85952 74.471197) (width 0.25) (layer "F.Cu") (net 15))
 (segment (start 99.865 76.415) (end 100.72452 77.27452) (width 0.25) (layer "F.Cu") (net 15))
 (segment (start 105.85952 70.02548) (end 106.68 69.205) (width 0.25) (layer "F.Cu") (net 15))
 (segment (start 127.645 69.205) (end 130.175 66.675) (width 0.25) (layer "F.Cu") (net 15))
 (segment (start 119.8875 73.015) (end 119.8875 76.14) (width 2) (layer "F.Cu") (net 18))
 (segment (start 119.8875 76.14) (end 119.595 76.4325) (width 2) (layer "F.Cu") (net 18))
 (segment (start 89.705 58.165) (end 89.705 52.65) (width 0.25) (layer "F.Cu") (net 46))
 (segment (start 87.63 50.575) (end 87.63 50.155) (width 0.25) (layer "F.Cu") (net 46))
 (segment (start 89.705 52.65) (end 87.63 50.575) (width 0.25) (layer "F.Cu") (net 46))
 (segment (start 90.17 50.155) (end 90.975 50.96) (width 0.25) (layer "F.Cu") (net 45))
 (segment (start 90.975 50.96) (end 90.975 58.165) (width 0.25) (layer "F.Cu") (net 45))
 (segment (start 88.435 75.994022) (end 90.545978 78.105) (width 0.25) (layer "F.Cu") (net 17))
 (segment (start 102.493533 60.175489) (end 101.739511 60.175489) (width 0.25) (layer "F.Cu") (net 17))
 (segment (start 104.775 57.894022) (end 102.493533 60.175489) (width 0.25) (layer "F.Cu") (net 17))
 (segment (start 88.435 74.335978) (end 88.435 75.165) (width 0.25) (layer "F.Cu") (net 17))
 (segment (start 104.775 53.19) (end 104.775 57.894022) (width 0.25) (layer "F.Cu") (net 17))
 (segment (start 94.335 80.6325) (end 94.3225 80.645) (width 0.25) (layer "F.Cu") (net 17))
 (segment (start 97.155 64.76) (end 97.155 71.11) (width 0.25) (layer "F.Cu") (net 17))
 (segment (start 94.335 78.105) (end 94.335 80.6325) (width 0.25) (layer "F.Cu") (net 17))
 (segment (start 90.525 78.084022) (end 90.525 78.095) (width 0.25) (layer "F.Cu") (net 17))
 (segment (start 90.390978 72.38) (end 88.435 74.335978) (width 0.25) (layer "F.Cu") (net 17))
 (segment (start 95.885 72.38) (end 90.390978 72.38) (width 0.25) (layer "F.Cu") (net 17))
 (segment (start 90.545978 78.105) (end 94.335 78.105) (width 0.25) (layer "F.Cu") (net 17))
 (segment (start 97.155 71.11) (end 95.885 72.38) (width 0.25) (layer "F.Cu") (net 17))
 (segment (start 101.739511 60.175489) (end 97.155 64.76) (width 0.25) (layer "F.Cu") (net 17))
 (segment (start 88.435 75.165) (end 88.435 75.994022) (width 0.25) (layer "F.Cu") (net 17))
 (segment (start 99.06 53.19) (end 102.405 56.535) (width 0.25) (layer "F.Cu") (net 36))
 (segment (start 102.405 56.535) (end 102.405 58.165) (width 0.25) (layer "F.Cu") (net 36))
 (segment (start 125.6675 84.735) (end 125.73 84.6725) (width 0.6) (layer "F.Cu") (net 16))
 (segment (start 123.19 84.735) (end 125.6675 84.735) (width 0.6) (layer "F.Cu") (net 16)))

